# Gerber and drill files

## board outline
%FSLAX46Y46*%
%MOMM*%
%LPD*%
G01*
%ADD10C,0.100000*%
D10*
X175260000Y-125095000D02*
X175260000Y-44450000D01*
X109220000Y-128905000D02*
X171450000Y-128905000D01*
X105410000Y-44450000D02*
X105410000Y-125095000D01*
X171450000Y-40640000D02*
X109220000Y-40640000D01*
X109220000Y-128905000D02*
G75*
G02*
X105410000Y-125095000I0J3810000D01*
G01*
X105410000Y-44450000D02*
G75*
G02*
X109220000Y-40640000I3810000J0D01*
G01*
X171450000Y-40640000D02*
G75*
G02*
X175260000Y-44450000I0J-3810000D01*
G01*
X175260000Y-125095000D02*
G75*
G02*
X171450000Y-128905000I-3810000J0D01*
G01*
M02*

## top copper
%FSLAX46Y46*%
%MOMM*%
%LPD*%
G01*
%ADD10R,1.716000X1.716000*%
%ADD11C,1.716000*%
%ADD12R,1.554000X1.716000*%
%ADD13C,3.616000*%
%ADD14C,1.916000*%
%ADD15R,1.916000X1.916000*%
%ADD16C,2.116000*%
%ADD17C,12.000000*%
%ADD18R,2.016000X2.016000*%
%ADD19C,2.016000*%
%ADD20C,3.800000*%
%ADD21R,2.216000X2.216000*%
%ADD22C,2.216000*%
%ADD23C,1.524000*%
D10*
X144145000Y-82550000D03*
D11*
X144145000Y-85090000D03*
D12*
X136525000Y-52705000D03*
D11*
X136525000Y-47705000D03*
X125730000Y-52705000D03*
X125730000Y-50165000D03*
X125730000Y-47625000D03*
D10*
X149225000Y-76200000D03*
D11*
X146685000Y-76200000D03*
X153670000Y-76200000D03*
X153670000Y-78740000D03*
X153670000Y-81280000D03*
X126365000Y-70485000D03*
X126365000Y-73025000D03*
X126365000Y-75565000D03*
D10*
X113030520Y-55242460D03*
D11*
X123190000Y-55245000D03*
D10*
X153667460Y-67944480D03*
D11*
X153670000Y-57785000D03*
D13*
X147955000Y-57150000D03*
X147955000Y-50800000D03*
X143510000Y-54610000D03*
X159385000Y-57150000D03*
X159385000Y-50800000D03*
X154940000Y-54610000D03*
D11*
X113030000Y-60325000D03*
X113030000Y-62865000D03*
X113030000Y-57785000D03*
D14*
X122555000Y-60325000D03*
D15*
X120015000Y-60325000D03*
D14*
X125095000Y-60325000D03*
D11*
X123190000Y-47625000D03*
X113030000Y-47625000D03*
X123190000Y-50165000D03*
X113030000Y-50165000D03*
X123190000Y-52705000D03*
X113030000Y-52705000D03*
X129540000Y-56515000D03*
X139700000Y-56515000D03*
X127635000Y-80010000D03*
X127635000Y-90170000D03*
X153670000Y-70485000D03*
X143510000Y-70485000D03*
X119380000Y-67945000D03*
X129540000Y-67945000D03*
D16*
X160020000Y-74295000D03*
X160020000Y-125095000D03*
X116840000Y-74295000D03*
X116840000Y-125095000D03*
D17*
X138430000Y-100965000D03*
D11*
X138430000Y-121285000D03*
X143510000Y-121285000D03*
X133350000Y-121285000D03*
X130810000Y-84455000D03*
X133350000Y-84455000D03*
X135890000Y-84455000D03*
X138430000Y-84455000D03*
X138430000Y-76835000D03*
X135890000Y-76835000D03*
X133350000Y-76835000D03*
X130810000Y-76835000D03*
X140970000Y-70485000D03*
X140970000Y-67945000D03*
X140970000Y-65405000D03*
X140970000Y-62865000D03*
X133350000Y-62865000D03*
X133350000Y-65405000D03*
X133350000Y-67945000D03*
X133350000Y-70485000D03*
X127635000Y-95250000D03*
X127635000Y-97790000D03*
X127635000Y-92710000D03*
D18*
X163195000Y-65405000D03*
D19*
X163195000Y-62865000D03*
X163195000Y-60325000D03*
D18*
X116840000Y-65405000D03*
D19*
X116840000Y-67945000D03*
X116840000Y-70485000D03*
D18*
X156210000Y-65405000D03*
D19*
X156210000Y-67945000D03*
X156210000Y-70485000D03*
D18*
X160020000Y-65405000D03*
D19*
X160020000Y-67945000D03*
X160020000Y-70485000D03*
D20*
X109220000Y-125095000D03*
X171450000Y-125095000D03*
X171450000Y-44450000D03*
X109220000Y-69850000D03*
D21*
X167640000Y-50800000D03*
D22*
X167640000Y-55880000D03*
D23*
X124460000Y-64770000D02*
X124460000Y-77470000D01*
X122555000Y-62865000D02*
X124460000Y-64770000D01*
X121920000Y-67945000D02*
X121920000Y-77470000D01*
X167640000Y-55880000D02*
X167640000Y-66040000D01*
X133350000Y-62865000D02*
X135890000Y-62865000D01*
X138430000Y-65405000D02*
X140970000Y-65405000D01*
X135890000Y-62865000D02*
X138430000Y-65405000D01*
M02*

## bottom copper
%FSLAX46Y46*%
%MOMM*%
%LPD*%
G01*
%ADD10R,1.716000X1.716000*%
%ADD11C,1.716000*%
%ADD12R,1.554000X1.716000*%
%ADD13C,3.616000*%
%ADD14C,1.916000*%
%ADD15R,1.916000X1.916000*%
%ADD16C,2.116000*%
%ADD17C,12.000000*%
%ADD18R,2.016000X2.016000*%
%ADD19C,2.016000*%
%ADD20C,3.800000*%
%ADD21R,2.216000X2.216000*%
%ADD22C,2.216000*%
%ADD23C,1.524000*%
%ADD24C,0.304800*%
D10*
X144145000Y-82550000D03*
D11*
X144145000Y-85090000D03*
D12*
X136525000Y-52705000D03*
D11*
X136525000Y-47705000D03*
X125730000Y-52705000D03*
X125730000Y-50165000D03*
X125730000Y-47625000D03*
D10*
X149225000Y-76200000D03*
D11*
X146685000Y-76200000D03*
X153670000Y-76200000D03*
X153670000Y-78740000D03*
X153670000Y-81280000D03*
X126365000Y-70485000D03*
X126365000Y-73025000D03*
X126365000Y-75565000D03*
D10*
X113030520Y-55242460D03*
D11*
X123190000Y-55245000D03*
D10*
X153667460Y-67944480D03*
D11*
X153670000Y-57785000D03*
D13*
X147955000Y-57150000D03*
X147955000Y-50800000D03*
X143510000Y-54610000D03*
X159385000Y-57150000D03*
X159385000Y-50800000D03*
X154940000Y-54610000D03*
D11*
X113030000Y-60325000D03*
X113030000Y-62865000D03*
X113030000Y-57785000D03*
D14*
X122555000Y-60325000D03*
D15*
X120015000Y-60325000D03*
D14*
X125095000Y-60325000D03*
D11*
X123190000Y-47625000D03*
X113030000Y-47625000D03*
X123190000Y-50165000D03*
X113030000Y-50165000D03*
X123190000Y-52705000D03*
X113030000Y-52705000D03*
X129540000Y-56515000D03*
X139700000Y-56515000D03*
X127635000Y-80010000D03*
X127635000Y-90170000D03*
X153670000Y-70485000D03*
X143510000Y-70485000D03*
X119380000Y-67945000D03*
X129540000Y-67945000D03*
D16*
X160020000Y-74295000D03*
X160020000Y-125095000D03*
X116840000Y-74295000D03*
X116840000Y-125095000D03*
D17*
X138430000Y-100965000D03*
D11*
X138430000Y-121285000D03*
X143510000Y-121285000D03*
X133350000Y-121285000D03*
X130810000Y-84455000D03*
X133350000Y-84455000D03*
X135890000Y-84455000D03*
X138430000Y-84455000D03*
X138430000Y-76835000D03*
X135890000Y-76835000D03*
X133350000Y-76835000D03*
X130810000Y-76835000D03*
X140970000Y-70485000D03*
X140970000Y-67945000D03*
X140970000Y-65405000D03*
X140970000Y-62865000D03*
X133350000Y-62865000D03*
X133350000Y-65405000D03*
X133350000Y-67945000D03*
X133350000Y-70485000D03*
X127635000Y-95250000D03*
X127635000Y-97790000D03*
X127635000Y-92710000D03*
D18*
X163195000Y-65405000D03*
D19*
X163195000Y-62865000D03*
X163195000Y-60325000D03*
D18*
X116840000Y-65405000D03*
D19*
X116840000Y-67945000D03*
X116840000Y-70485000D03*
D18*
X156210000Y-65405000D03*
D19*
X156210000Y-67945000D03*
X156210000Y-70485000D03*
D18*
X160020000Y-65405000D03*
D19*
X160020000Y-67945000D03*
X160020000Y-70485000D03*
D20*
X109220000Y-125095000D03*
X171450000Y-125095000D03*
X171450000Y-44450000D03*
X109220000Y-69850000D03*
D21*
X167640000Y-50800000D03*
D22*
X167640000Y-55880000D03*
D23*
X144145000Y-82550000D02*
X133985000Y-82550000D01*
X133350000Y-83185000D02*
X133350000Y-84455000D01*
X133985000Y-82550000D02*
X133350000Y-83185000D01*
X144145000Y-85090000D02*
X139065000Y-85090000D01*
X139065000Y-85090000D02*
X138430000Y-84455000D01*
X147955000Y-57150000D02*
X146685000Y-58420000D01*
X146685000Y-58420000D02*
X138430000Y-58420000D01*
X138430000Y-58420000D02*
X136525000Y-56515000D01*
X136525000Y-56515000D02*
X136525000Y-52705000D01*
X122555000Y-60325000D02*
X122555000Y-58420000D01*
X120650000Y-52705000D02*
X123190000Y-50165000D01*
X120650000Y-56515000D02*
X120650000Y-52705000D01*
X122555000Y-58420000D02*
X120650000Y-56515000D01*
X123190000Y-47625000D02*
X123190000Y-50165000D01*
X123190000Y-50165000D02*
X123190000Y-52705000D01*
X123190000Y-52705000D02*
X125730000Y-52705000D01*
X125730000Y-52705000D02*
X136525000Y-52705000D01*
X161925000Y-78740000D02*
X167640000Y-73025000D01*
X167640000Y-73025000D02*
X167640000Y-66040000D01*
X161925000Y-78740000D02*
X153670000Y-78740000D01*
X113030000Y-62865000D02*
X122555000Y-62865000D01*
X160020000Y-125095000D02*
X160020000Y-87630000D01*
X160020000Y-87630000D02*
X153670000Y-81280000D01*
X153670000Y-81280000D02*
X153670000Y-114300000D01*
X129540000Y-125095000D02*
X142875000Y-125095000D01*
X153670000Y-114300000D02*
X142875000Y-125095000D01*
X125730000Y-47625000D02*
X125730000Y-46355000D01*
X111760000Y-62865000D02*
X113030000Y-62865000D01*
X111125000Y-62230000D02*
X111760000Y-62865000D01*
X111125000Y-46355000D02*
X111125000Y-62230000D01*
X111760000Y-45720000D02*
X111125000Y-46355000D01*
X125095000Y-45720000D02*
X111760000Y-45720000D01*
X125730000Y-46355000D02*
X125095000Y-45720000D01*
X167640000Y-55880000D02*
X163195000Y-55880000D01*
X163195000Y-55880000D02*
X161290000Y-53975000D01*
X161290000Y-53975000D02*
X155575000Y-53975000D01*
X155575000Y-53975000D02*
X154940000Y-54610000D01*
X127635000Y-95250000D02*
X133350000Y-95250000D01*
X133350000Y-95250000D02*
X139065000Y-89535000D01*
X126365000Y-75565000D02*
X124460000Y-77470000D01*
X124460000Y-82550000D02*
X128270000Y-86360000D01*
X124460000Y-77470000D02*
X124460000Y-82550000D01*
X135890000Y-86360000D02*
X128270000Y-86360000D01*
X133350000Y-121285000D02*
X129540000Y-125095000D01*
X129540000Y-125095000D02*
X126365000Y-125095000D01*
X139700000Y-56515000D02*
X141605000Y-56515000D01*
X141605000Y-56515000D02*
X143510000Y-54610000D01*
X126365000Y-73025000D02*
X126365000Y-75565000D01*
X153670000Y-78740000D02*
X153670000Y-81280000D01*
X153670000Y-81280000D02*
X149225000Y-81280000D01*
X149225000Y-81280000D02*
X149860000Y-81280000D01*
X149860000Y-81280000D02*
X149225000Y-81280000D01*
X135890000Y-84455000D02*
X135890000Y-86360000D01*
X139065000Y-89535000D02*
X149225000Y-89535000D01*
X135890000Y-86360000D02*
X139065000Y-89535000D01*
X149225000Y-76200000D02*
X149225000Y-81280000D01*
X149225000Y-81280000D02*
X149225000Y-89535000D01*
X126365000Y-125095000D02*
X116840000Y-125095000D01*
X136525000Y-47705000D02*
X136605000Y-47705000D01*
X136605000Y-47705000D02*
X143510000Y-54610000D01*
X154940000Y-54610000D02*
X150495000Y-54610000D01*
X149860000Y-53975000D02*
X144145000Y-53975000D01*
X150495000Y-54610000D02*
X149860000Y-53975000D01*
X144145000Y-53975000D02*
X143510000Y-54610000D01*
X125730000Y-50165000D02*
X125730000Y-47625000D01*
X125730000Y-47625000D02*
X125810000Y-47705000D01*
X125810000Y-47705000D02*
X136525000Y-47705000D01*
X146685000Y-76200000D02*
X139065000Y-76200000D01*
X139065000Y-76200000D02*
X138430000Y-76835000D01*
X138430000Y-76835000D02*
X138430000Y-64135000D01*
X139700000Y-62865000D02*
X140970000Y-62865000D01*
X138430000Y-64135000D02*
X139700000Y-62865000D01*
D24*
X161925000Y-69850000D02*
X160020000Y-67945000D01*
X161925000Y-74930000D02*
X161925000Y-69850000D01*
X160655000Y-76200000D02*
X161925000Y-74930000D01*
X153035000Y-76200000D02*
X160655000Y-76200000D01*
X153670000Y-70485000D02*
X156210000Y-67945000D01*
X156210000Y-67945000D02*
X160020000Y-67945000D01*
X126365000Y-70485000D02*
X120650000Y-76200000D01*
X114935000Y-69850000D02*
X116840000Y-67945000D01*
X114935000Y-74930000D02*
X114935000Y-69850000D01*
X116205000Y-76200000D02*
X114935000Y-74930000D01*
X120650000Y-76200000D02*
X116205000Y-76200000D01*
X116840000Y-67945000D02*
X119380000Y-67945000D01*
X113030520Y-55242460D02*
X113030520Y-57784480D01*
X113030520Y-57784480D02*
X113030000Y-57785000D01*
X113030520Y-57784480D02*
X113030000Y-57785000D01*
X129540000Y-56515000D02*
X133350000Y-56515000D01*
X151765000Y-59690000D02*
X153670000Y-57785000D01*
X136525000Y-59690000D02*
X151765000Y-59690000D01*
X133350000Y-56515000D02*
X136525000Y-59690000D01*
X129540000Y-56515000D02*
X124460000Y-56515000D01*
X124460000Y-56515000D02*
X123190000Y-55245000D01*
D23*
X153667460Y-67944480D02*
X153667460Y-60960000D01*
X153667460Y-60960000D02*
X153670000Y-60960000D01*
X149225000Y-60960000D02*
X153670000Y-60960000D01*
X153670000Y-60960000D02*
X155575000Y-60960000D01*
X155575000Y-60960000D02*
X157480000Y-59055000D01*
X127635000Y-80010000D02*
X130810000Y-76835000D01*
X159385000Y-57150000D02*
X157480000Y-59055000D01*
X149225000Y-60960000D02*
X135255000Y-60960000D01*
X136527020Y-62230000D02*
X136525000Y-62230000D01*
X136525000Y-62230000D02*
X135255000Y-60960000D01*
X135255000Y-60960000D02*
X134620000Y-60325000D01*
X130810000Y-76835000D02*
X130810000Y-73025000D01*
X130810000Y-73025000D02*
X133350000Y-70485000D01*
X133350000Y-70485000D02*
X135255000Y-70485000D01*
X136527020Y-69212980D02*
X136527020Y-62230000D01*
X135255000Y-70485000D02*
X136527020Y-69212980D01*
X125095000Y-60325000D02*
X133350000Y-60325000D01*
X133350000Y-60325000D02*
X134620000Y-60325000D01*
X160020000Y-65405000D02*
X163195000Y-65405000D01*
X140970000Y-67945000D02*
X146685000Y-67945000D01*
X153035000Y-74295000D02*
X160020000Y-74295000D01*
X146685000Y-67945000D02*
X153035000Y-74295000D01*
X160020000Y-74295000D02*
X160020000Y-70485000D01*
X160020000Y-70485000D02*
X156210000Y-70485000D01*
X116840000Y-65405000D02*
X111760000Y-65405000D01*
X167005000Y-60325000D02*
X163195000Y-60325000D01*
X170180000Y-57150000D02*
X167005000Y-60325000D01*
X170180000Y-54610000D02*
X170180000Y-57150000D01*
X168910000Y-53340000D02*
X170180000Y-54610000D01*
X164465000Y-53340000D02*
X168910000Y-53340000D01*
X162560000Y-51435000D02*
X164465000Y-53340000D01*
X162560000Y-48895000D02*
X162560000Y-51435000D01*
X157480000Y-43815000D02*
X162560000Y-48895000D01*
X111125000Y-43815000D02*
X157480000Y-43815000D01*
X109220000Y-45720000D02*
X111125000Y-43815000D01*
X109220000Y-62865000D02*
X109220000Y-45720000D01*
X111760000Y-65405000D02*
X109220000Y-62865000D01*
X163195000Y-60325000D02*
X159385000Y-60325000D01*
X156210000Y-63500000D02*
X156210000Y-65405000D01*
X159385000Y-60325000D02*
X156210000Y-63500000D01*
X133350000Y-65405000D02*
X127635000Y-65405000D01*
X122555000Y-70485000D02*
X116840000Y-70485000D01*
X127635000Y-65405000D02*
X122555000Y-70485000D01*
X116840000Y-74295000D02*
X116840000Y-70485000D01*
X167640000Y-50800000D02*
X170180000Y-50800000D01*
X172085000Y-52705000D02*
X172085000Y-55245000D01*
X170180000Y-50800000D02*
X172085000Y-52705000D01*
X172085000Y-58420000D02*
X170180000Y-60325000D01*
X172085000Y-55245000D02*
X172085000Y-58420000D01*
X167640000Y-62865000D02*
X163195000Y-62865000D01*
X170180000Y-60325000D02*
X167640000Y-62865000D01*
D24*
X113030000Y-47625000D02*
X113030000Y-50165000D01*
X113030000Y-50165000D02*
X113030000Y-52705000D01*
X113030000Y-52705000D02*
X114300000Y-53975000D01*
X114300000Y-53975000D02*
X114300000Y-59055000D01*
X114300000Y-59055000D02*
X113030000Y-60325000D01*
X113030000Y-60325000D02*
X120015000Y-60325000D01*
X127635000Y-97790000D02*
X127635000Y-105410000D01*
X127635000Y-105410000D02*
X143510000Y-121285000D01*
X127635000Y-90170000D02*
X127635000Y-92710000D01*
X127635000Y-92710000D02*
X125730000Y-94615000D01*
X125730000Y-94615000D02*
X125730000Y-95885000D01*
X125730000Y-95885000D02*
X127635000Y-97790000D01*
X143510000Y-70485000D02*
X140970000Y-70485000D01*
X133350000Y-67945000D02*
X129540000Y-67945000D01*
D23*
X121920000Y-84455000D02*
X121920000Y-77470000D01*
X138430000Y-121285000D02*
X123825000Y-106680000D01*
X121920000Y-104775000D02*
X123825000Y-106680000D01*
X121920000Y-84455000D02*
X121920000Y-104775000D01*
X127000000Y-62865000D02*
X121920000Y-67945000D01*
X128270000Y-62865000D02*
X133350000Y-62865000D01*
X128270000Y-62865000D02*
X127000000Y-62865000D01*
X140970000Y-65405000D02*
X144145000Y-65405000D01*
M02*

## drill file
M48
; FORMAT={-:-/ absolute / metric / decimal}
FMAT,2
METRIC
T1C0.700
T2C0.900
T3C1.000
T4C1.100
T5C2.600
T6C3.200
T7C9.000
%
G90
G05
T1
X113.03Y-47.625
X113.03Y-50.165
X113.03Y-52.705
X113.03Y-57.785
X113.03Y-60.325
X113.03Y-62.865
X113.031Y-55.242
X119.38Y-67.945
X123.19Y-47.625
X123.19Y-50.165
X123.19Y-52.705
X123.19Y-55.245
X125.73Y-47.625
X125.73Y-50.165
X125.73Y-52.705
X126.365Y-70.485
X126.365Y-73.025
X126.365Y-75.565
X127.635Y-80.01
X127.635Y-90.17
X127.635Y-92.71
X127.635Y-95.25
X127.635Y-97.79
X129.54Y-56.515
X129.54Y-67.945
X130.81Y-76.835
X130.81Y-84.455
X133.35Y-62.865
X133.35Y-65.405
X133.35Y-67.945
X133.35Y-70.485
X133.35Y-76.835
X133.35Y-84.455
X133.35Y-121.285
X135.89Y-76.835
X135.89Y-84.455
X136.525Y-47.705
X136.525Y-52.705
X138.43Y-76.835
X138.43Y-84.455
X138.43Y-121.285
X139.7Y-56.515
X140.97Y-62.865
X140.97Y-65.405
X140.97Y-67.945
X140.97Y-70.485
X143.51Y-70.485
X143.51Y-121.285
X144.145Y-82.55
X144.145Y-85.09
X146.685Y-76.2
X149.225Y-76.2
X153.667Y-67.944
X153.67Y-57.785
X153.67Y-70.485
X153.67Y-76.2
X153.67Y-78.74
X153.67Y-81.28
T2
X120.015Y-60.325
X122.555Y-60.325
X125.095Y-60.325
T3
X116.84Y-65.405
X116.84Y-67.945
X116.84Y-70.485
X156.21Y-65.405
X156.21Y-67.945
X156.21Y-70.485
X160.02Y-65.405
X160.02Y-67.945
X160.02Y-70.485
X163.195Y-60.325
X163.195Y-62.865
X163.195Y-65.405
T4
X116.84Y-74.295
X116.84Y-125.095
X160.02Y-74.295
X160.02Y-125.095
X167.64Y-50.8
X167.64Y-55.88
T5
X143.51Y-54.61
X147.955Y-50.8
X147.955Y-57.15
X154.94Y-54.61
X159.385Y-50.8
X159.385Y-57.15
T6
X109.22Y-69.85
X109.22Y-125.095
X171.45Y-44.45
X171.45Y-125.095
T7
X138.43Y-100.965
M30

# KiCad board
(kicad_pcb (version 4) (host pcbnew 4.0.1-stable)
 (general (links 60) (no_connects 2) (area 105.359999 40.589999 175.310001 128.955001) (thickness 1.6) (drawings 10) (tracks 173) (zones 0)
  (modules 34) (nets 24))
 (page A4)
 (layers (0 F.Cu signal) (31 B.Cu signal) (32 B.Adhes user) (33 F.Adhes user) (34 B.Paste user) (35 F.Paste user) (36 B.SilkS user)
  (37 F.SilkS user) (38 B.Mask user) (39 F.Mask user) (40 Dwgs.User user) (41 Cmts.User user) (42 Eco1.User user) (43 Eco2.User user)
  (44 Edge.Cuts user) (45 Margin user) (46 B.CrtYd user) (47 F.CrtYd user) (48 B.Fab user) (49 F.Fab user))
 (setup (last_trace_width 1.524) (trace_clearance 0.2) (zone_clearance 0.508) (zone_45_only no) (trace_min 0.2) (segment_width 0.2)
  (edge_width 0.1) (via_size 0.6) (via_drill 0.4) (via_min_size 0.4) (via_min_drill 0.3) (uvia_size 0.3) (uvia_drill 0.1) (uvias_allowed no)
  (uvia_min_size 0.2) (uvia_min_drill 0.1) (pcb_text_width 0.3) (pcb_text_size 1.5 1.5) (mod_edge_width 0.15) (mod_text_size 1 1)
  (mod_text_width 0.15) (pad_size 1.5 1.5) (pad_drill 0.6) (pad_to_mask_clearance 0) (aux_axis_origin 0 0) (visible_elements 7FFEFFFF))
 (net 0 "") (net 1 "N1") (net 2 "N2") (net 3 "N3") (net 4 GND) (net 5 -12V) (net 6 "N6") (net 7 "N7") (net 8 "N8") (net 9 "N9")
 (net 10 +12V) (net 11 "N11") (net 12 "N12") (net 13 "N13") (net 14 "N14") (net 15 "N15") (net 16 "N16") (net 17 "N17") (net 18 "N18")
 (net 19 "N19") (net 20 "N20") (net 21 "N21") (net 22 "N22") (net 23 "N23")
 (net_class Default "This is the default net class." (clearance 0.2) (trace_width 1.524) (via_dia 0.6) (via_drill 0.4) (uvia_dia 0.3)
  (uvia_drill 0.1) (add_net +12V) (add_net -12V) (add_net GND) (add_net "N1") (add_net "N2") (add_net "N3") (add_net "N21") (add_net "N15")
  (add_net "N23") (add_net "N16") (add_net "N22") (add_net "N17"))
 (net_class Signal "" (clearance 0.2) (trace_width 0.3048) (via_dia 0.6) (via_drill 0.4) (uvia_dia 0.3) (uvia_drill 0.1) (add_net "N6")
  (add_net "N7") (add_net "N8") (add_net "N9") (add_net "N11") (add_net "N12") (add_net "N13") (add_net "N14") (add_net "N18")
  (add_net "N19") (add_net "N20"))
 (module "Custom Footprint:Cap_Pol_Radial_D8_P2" (layer F.Cu) (at 144.145 82.55 270)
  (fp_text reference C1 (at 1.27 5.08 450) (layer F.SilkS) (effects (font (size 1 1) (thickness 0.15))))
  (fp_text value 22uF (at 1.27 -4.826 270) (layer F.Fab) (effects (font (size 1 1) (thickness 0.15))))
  (pad 1 thru_hole rect (at 0 0 270) (size 1.716 1.716) (drill 0.7) (layers *.Cu *.Mask F.SilkS) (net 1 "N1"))
  (pad 2 thru_hole circle (at 2.54 0 270) (size 1.716 1.716) (drill 0.7) (layers *.Cu *.Mask F.SilkS) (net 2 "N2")))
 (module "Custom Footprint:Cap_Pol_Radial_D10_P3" (layer F.Cu) (at 136.525 52.705 90)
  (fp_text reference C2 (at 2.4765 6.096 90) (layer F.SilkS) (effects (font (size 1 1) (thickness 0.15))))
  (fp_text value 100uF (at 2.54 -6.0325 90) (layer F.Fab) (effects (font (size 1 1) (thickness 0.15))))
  (pad 1 thru_hole rect (at 0 0 90) (size 1.716 1.554) (drill 0.7) (layers *.Cu *.Mask F.SilkS) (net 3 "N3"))
  (pad 2 thru_hole circle (at 5 0 90) (size 1.716 1.716) (drill 0.7) (layers *.Cu *.Mask F.SilkS) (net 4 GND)))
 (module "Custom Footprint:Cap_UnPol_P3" (layer F.Cu) (at 125.73 52.705 180)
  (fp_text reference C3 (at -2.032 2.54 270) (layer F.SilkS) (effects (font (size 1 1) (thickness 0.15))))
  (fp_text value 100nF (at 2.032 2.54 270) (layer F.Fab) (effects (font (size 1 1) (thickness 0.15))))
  (pad 1 thru_hole circle (at 0 0 180) (size 1.716 1.716) (drill 0.7) (layers *.Cu *.Mask F.SilkS) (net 3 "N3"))
  (pad 2 thru_hole circle (at 0 2.54 180) (size 1.716 1.716) (drill 0.7) (layers *.Cu *.Mask F.SilkS) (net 4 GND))
  (pad 2 thru_hole circle (at 0 5.08 180) (size 1.716 1.716) (drill 0.7) (layers *.Cu *.Mask F.SilkS) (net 4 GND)))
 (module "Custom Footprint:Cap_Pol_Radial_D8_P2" (layer F.Cu) (at 149.225 76.2 180)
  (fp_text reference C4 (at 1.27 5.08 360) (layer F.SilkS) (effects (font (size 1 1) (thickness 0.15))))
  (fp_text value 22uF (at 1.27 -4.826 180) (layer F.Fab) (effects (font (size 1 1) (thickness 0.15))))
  (pad 1 thru_hole rect (at 0 0 180) (size 1.716 1.716) (drill 0.7) (layers *.Cu *.Mask F.SilkS) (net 4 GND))
  (pad 2 thru_hole circle (at 2.54 0 180) (size 1.716 1.716) (drill 0.7) (layers *.Cu *.Mask F.SilkS) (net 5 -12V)))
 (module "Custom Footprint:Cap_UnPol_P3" (layer F.Cu) (at 153.67 76.2)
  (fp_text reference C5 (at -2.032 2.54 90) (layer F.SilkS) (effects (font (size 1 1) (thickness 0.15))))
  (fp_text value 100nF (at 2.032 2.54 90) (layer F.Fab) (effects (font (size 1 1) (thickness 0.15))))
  (pad 1 thru_hole circle (at 0 0) (size 1.716 1.716) (drill 0.7) (layers *.Cu *.Mask F.SilkS) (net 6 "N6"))
  (pad 2 thru_hole circle (at 0 2.54) (size 1.716 1.716) (drill 0.7) (layers *.Cu *.Mask F.SilkS) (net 4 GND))
  (pad 2 thru_hole circle (at 0 5.08) (size 1.716 1.716) (drill 0.7) (layers *.Cu *.Mask F.SilkS) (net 4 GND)))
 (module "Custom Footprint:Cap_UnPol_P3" (layer F.Cu) (at 126.365 70.485)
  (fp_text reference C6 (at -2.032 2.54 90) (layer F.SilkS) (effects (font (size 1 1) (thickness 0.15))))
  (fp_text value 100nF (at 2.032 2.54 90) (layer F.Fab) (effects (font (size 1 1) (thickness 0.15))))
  (pad 1 thru_hole circle (at 0 0) (size 1.716 1.716) (drill 0.7) (layers *.Cu *.Mask F.SilkS) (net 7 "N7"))
  (pad 2 thru_hole circle (at 0 2.54) (size 1.716 1.716) (drill 0.7) (layers *.Cu *.Mask F.SilkS) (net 4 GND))
  (pad 2 thru_hole circle (at 0 5.08) (size 1.716 1.716) (drill 0.7) (layers *.Cu *.Mask F.SilkS) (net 4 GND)))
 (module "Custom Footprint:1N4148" (layer F.Cu) (at 113.03 55.245)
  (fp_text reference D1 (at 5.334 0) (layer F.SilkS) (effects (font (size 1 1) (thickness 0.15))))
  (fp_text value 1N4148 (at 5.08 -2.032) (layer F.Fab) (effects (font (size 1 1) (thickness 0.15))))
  (pad 1 thru_hole rect (at 0.00052 -0.00254 180) (size 1.716 1.716) (drill 0.7) (layers *.Cu *.Mask F.SilkS) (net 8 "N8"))
  (pad 2 thru_hole circle (at 10.16 0) (size 1.716 1.716) (drill 0.7) (layers *.Cu *.Mask F.SilkS) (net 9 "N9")))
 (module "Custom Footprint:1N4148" (layer F.Cu) (at 153.67 67.945 90)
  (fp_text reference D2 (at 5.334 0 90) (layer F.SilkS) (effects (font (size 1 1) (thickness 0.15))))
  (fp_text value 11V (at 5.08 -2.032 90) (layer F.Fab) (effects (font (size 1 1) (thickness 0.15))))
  (pad 1 thru_hole rect (at 0.00052 -0.00254 270) (size 1.716 1.716) (drill 0.7) (layers *.Cu *.Mask F.SilkS) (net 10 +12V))
  (pad 2 thru_hole circle (at 10.16 0 90) (size 1.716 1.716) (drill 0.7) (layers *.Cu *.Mask F.SilkS) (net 9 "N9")))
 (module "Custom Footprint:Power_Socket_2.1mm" (layer F.Cu) (at 147.955 50.8)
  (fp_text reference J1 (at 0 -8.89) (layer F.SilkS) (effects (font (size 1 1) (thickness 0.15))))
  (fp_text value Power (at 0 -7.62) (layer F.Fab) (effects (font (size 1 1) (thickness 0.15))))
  (pad 1 thru_hole circle (at 0 6.35) (size 3.616 3.616) (drill 2.6) (layers *.Cu *.Mask F.SilkS) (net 3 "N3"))
  (pad 3 thru_hole circle (at 0 0) (size 3.616 3.616) (drill 2.6) (layers *.Cu *.Mask F.SilkS))
  (pad 2 thru_hole circle (at -4.445 3.81) (size 3.616 3.616) (drill 2.6) (layers *.Cu *.Mask F.SilkS) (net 4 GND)))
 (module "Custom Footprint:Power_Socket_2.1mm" (layer F.Cu) (at 159.385 50.8)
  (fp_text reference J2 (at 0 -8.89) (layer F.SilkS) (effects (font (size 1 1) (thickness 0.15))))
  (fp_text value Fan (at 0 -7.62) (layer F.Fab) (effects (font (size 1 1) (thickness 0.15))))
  (pad 1 thru_hole circle (at 0 6.35) (size 3.616 3.616) (drill 2.6) (layers *.Cu *.Mask F.SilkS) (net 10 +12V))
  (pad 3 thru_hole circle (at 0 0) (size 3.616 3.616) (drill 2.6) (layers *.Cu *.Mask F.SilkS))
  (pad 2 thru_hole circle (at -4.445 3.81) (size 3.616 3.616) (drill 2.6) (layers *.Cu *.Mask F.SilkS) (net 4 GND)))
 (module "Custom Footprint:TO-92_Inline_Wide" (layer F.Cu) (at 113.03 57.785 270)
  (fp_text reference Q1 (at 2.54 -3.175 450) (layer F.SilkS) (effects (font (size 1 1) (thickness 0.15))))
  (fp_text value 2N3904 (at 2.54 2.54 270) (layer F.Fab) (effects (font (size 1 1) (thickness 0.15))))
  (pad 2 thru_hole circle (at 2.54 0) (size 1.716 1.716) (drill 0.7) (layers *.Cu *.Mask F.SilkS) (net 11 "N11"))
  (pad 3 thru_hole circle (at 5.08 0) (size 1.716 1.716) (drill 0.7) (layers *.Cu *.Mask F.SilkS) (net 4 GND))
  (pad 1 thru_hole circle (at 0 0) (size 1.716 1.716) (drill 0.7) (layers *.Cu *.Mask F.SilkS) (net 8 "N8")))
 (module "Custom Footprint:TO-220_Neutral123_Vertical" (layer F.Cu) (at 122.555 60.325)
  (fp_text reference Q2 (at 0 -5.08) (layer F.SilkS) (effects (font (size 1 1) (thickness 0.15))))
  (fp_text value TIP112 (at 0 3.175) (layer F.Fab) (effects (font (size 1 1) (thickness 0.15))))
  (pad 2 thru_hole circle (at 0 0 90) (size 1.916 1.916) (drill 0.9) (layers *.Cu *.Mask F.SilkS) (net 3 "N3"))
  (pad 1 thru_hole rect (at -2.54 0 90) (size 1.916 1.916) (drill 0.9) (layers *.Cu *.Mask F.SilkS) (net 11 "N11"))
  (pad 3 thru_hole circle (at 2.54 0 90) (size 1.916 1.916) (drill 0.9) (layers *.Cu *.Mask F.SilkS) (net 10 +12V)))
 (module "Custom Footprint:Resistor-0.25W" (layer F.Cu) (at 123.19 47.625 180)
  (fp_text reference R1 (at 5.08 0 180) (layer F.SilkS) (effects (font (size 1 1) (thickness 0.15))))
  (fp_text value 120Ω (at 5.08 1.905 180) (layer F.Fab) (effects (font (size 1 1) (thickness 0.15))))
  (pad 1 thru_hole circle (at 0 0 180) (size 1.716 1.716) (drill 0.7) (layers *.Cu *.Mask F.SilkS) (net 3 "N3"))
  (pad 2 thru_hole circle (at 10.16 0 180) (size 1.716 1.716) (drill 0.7) (layers *.Cu *.Mask F.SilkS) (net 11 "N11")))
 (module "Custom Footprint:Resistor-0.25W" (layer F.Cu) (at 123.19 50.165 180)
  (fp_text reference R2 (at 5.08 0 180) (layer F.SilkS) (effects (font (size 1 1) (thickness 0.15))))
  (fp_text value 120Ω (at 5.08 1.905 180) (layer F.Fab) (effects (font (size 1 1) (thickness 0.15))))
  (pad 1 thru_hole circle (at 0 0 180) (size 1.716 1.716) (drill 0.7) (layers *.Cu *.Mask F.SilkS) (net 3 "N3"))
  (pad 2 thru_hole circle (at 10.16 0 180) (size 1.716 1.716) (drill 0.7) (layers *.Cu *.Mask F.SilkS) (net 11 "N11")))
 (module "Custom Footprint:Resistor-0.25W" (layer F.Cu) (at 123.19 52.705 180)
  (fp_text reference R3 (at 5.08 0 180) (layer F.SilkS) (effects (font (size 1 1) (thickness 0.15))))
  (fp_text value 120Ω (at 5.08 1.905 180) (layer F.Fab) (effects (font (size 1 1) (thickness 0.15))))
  (pad 1 thru_hole circle (at 0 0 180) (size 1.716 1.716) (drill 0.7) (layers *.Cu *.Mask F.SilkS) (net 3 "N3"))
  (pad 2 thru_hole circle (at 10.16 0 180) (size 1.716 1.716) (drill 0.7) (layers *.Cu *.Mask F.SilkS) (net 11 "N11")))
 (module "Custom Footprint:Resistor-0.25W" (layer F.Cu) (at 129.54 56.515)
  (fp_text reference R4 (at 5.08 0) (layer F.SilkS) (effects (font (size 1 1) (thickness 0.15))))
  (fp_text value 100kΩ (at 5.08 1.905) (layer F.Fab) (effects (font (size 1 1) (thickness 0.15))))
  (pad 1 thru_hole circle (at 0 0) (size 1.716 1.716) (drill 0.7) (layers *.Cu *.Mask F.SilkS) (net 9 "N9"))
  (pad 2 thru_hole circle (at 10.16 0) (size 1.716 1.716) (drill 0.7) (layers *.Cu *.Mask F.SilkS) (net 4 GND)))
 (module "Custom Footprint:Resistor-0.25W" (layer F.Cu) (at 127.635 80.01 270)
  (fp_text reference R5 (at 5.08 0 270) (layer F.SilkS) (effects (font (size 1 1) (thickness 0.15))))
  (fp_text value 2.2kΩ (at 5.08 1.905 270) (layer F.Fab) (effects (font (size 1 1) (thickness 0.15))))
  (pad 1 thru_hole circle (at 0 0 270) (size 1.716 1.716) (drill 0.7) (layers *.Cu *.Mask F.SilkS) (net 10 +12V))
  (pad 2 thru_hole circle (at 10.16 0 270) (size 1.716 1.716) (drill 0.7) (layers *.Cu *.Mask F.SilkS) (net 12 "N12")))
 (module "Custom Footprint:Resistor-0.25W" (layer F.Cu) (at 153.67 70.485 180)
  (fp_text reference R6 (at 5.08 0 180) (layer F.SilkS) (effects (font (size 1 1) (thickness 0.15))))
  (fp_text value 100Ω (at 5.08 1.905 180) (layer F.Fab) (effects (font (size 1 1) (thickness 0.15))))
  (pad 1 thru_hole circle (at 0 0 180) (size 1.716 1.716) (drill 0.7) (layers *.Cu *.Mask F.SilkS) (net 6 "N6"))
  (pad 2 thru_hole circle (at 10.16 0 180) (size 1.716 1.716) (drill 0.7) (layers *.Cu *.Mask F.SilkS) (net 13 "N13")))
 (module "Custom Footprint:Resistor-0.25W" (layer F.Cu) (at 119.38 67.945)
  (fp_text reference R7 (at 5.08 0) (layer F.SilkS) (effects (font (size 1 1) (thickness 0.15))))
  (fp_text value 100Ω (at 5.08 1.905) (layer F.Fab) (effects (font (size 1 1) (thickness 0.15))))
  (pad 1 thru_hole circle (at 0 0) (size 1.716 1.716) (drill 0.7) (layers *.Cu *.Mask F.SilkS) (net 7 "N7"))
  (pad 2 thru_hole circle (at 10.16 0) (size 1.716 1.716) (drill 0.7) (layers *.Cu *.Mask F.SilkS) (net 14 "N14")))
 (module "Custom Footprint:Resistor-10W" (layer F.Cu) (at 160.02 99.695 270)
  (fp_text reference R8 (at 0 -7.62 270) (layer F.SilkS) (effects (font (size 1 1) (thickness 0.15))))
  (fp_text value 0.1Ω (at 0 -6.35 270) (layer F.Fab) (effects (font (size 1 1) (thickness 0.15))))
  (pad 1 thru_hole circle (at -25.4 0 270) (size 2.116 2.116) (drill 1.1) (layers *.Cu *.Mask F.SilkS) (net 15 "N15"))
  (pad 2 thru_hole circle (at 25.4 0 270) (size 2.116 2.116) (drill 1.1) (layers *.Cu *.Mask F.SilkS) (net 4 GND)))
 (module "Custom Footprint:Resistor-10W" (layer F.Cu) (at 116.84 99.695 270)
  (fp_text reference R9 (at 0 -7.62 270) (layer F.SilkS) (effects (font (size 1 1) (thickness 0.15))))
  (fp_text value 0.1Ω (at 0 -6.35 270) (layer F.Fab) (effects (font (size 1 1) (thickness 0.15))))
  (pad 1 thru_hole circle (at -25.4 0 270) (size 2.116 2.116) (drill 1.1) (layers *.Cu *.Mask F.SilkS) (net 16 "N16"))
  (pad 2 thru_hole circle (at 25.4 0 270) (size 2.116 2.116) (drill 1.1) (layers *.Cu *.Mask F.SilkS) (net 4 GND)))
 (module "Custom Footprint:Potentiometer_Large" (layer F.Cu) (at 138.43 100.965)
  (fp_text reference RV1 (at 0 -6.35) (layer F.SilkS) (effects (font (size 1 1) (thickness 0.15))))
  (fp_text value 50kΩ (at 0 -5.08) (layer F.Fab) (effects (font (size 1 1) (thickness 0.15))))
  (pad "" thru_hole circle (at 0 0) (size 12 12) (drill 9) (layers *.Cu *.Mask F.SilkS))
  (pad 2 thru_hole circle (at 0 20.32) (size 1.716 1.716) (drill 0.7) (layers *.Cu *.Mask F.SilkS) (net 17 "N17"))
  (pad 3 thru_hole circle (at 5.08 20.32) (size 1.716 1.716) (drill 0.7) (layers *.Cu *.Mask F.SilkS) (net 12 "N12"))
  (pad 1 thru_hole circle (at -5.08 20.32) (size 1.716 1.716) (drill 0.7) (layers *.Cu *.Mask F.SilkS) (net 4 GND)))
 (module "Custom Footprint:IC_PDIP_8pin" (layer F.Cu) (at 134.62 80.645)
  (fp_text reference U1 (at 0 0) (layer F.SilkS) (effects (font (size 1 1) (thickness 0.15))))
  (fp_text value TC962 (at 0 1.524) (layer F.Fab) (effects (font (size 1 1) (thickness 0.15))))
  (pad 1 thru_hole circle (at -3.81 3.81) (size 1.716 1.716) (drill 0.7) (layers *.Cu *.Mask F.SilkS) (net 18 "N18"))
  (pad 2 thru_hole circle (at -1.27 3.81) (size 1.716 1.716) (drill 0.7) (layers *.Cu *.Mask F.SilkS) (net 1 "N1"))
  (pad 3 thru_hole circle (at 1.27 3.81) (size 1.716 1.716) (drill 0.7) (layers *.Cu *.Mask F.SilkS) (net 4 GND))
  (pad 4 thru_hole circle (at 3.81 3.81) (size 1.716 1.716) (drill 0.7) (layers *.Cu *.Mask F.SilkS) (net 2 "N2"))
  (pad 5 thru_hole circle (at 3.81 -3.81) (size 1.716 1.716) (drill 0.7) (layers *.Cu *.Mask F.SilkS) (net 5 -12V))
  (pad 6 thru_hole circle (at 1.27 -3.81) (size 1.716 1.716) (drill 0.7) (layers *.Cu *.Mask F.SilkS) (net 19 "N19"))
  (pad 7 thru_hole circle (at -1.27 -3.81) (size 1.716 1.716) (drill 0.7) (layers *.Cu *.Mask F.SilkS) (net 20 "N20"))
  (pad 8 thru_hole circle (at -3.81 -3.81) (size 1.716 1.716) (drill 0.7) (layers *.Cu *.Mask F.SilkS) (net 10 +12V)))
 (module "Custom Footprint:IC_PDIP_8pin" (layer F.Cu) (at 137.16 66.675 90)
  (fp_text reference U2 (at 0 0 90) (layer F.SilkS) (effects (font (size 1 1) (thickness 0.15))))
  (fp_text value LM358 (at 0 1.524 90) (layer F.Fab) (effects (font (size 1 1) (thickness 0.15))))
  (pad 1 thru_hole circle (at -3.81 3.81 90) (size 1.716 1.716) (drill 0.7) (layers *.Cu *.Mask F.SilkS) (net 13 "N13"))
  (pad 2 thru_hole circle (at -1.27 3.81 90) (size 1.716 1.716) (drill 0.7) (layers *.Cu *.Mask F.SilkS) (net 15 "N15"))
  (pad 3 thru_hole circle (at 1.27 3.81 90) (size 1.716 1.716) (drill 0.7) (layers *.Cu *.Mask F.SilkS) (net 17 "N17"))
  (pad 4 thru_hole circle (at 3.81 3.81 90) (size 1.716 1.716) (drill 0.7) (layers *.Cu *.Mask F.SilkS) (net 5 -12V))
  (pad 5 thru_hole circle (at 3.81 -3.81 90) (size 1.716 1.716) (drill 0.7) (layers *.Cu *.Mask F.SilkS) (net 17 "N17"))
  (pad 6 thru_hole circle (at 1.27 -3.81 90) (size 1.716 1.716) (drill 0.7) (layers *.Cu *.Mask F.SilkS) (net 16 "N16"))
  (pad 7 thru_hole circle (at -1.27 -3.81 90) (size 1.716 1.716) (drill 0.7) (layers *.Cu *.Mask F.SilkS) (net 14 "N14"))
  (pad 8 thru_hole circle (at -3.81 -3.81 90) (size 1.716 1.716) (drill 0.7) (layers *.Cu *.Mask F.SilkS) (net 10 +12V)))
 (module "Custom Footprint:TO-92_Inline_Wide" (layer F.Cu) (at 127.635 92.71 270)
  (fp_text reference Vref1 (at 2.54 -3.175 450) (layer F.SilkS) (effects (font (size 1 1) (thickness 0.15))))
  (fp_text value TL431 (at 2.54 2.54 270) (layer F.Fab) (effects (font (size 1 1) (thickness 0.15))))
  (pad 2 thru_hole circle (at 2.54 0) (size 1.716 1.716) (drill 0.7) (layers *.Cu *.Mask F.SilkS) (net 4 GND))
  (pad 3 thru_hole circle (at 5.08 0) (size 1.716 1.716) (drill 0.7) (layers *.Cu *.Mask F.SilkS) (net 12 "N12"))
  (pad 1 thru_hole circle (at 0 0) (size 1.716 1.716) (drill 0.7) (layers *.Cu *.Mask F.SilkS) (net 12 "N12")))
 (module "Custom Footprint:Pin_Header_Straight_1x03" (layer F.Cu) (at 163.195 65.405 180)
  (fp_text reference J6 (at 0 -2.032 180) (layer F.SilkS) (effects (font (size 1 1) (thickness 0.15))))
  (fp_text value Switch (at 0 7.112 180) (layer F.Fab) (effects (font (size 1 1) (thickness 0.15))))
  (pad 1 thru_hole rect (at 0 0 180) (size 2.016 2.016) (drill 1) (layers *.Cu *.Mask F.SilkS) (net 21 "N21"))
  (pad 2 thru_hole circle (at 0 2.54 180) (size 2.016 2.016) (drill 1) (layers *.Cu *.Mask F.SilkS) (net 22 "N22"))
  (pad 3 thru_hole circle (at 0 5.08 180) (size 2.016 2.016) (drill 1) (layers *.Cu *.Mask F.SilkS) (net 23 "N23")))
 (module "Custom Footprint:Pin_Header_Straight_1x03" (layer F.Cu) (at 116.84 65.405)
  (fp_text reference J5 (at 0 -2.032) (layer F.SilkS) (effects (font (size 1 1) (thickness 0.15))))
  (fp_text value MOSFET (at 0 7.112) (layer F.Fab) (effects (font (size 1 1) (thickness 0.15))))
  (pad 1 thru_hole rect (at 0 0) (size 2.016 2.016) (drill 1) (layers *.Cu *.Mask F.SilkS) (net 23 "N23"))
  (pad 2 thru_hole circle (at 0 2.54) (size 2.016 2.016) (drill 1) (layers *.Cu *.Mask F.SilkS) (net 7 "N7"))
  (pad 3 thru_hole circle (at 0 5.08) (size 2.016 2.016) (drill 1) (layers *.Cu *.Mask F.SilkS) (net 16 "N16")))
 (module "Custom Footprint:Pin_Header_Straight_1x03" (layer F.Cu) (at 156.21 65.405)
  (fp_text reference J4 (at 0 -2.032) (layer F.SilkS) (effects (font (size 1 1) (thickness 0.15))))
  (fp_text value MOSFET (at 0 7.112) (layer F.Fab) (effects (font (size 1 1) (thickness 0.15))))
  (pad 1 thru_hole rect (at 0 0) (size 2.016 2.016) (drill 1) (layers *.Cu *.Mask F.SilkS) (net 23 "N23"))
  (pad 2 thru_hole circle (at 0 2.54) (size 2.016 2.016) (drill 1) (layers *.Cu *.Mask F.SilkS) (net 6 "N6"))
  (pad 3 thru_hole circle (at 0 5.08) (size 2.016 2.016) (drill 1) (layers *.Cu *.Mask F.SilkS) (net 15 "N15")))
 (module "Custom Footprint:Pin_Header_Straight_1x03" (layer F.Cu) (at 160.02 65.405)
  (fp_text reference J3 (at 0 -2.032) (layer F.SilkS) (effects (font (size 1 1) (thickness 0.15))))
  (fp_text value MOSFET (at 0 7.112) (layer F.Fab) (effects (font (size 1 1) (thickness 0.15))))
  (pad 1 thru_hole rect (at 0 0) (size 2.016 2.016) (drill 1) (layers *.Cu *.Mask F.SilkS) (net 21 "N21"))
  (pad 2 thru_hole circle (at 0 2.54) (size 2.016 2.016) (drill 1) (layers *.Cu *.Mask F.SilkS) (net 6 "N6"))
  (pad 3 thru_hole circle (at 0 5.08) (size 2.016 2.016) (drill 1) (layers *.Cu *.Mask F.SilkS) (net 15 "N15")))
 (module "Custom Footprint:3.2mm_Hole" (layer F.Cu) (at 109.22 125.095)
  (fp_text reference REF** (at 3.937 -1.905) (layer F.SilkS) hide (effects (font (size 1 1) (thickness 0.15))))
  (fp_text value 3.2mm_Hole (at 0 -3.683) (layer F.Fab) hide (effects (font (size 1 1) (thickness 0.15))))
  (pad 1 thru_hole circle (at 0 0) (size 3.8 3.8) (drill 3.2) (layers *.Cu *.Mask F.SilkS)))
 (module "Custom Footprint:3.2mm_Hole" (layer F.Cu) (at 171.45 125.095)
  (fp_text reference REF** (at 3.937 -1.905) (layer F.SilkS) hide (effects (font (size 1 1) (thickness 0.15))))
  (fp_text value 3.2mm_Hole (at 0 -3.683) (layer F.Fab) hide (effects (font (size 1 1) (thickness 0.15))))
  (pad 1 thru_hole circle (at 0 0) (size 3.8 3.8) (drill 3.2) (layers *.Cu *.Mask F.SilkS)))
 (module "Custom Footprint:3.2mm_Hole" (layer F.Cu) (at 171.45 44.45)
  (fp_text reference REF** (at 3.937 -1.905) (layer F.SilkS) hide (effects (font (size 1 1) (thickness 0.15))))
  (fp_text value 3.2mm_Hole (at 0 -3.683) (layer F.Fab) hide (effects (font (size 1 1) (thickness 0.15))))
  (pad 1 thru_hole circle (at 0 0) (size 3.8 3.8) (drill 3.2) (layers *.Cu *.Mask F.SilkS)))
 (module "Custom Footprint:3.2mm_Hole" (layer F.Cu) (at 109.22 69.85)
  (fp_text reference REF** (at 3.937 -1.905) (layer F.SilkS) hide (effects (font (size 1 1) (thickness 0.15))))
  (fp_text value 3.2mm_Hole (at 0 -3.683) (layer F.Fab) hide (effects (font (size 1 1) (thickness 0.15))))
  (pad 1 thru_hole circle (at 0 0) (size 3.8 3.8) (drill 3.2) (layers *.Cu *.Mask F.SilkS)))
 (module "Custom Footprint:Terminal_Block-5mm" (layer F.Cu) (at 167.64 53.34 270)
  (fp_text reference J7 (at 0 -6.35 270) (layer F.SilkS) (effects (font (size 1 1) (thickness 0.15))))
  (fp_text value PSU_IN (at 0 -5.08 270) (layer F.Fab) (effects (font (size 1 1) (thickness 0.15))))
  (pad 1 thru_hole rect (at -2.54 0 270) (size 2.216 2.216) (drill 1.1) (layers *.Cu *.Mask F.SilkS) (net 22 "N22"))
  (pad 2 thru_hole circle (at 2.54 0 270) (size 2.216 2.216) (drill 1.1) (layers *.Cu *.Mask F.SilkS) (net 4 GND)))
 (gr_line (start 175.26 125.095) (end 175.26 44.45) (angle 90) (layer Edge.Cuts) (width 0.1))
 (gr_line (start 109.22 128.905) (end 171.45 128.905) (angle 90) (layer Edge.Cuts) (width 0.1))
 (gr_line (start 105.41 44.45) (end 105.41 125.095) (angle 90) (layer Edge.Cuts) (width 0.1))
 (gr_line (start 171.45 40.64) (end 109.22 40.64) (angle 90) (layer Edge.Cuts) (width 0.1))
 (gr_arc (start 109.22 125.095) (end 109.22 128.905) (angle 90) (layer Edge.Cuts) (width 0.1))
 (gr_arc (start 109.22 44.45) (end 105.41 44.45) (angle 90) (layer Edge.Cuts) (width 0.1))
 (gr_arc (start 171.45 44.45) (end 171.45 40.64) (angle 90) (layer Edge.Cuts) (width 0.1))
 (gr_arc (start 171.45 125.095) (end 175.26 125.095) (angle 90) (layer Edge.Cuts) (width 0.1))
 (segment (start 124.46 64.77) (end 124.46 77.47) (width 1.524) (layer F.Cu) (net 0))
 (segment (start 122.555 62.865) (end 124.46 64.77) (width 1.524) (layer F.Cu) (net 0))
 (segment (start 121.92 67.945) (end 121.92 77.47) (width 1.524) (layer F.Cu) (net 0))
 (segment (start 144.145 82.55) (end 133.985 82.55) (width 1.524) (layer B.Cu) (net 1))
 (segment (start 133.35 83.185) (end 133.35 84.455) (width 1.524) (layer B.Cu) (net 1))
 (segment (start 133.985 82.55) (end 133.35 83.185) (width 1.524) (layer B.Cu) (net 1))
 (segment (start 144.145 85.09) (end 139.065 85.09) (width 1.524) (layer B.Cu) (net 2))
 (segment (start 139.065 85.09) (end 138.43 84.455) (width 1.524) (layer B.Cu) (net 2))
 (segment (start 147.955 57.15) (end 146.685 58.42) (width 1.524) (layer B.Cu) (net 3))
 (segment (start 146.685 58.42) (end 138.43 58.42) (width 1.524) (layer B.Cu) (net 3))
 (segment (start 138.43 58.42) (end 136.525 56.515) (width 1.524) (layer B.Cu) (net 3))
 (segment (start 136.525 56.515) (end 136.525 52.705) (width 1.524) (layer B.Cu) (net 3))
 (segment (start 122.555 60.325) (end 122.555 58.42) (width 1.524) (layer B.Cu) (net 3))
 (segment (start 120.65 52.705) (end 123.19 50.165) (width 1.524) (layer B.Cu) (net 3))
 (segment (start 120.65 56.515) (end 120.65 52.705) (width 1.524) (layer B.Cu) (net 3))
 (segment (start 122.555 58.42) (end 120.65 56.515) (width 1.524) (layer B.Cu) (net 3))
 (segment (start 123.19 47.625) (end 123.19 50.165) (width 1.524) (layer B.Cu) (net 3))
 (segment (start 123.19 50.165) (end 123.19 52.705) (width 1.524) (layer B.Cu) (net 3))
 (segment (start 123.19 52.705) (end 125.73 52.705) (width 1.524) (layer B.Cu) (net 3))
 (segment (start 125.73 52.705) (end 136.525 52.705) (width 1.524) (layer B.Cu) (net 3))
 (segment (start 167.64 55.88) (end 167.64 66.04) (width 1.524) (layer F.Cu) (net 4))
 (segment (start 161.925 78.74) (end 167.64 73.025) (width 1.524) (layer B.Cu) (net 4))
 (segment (start 167.64 73.025) (end 167.64 66.04) (width 1.524) (layer B.Cu) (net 4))
 (segment (start 161.925 78.74) (end 153.67 78.74) (width 1.524) (layer B.Cu) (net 4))
 (segment (start 113.03 62.865) (end 122.555 62.865) (width 1.524) (layer B.Cu) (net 4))
 (segment (start 160.02 125.095) (end 160.02 87.63) (width 1.524) (layer B.Cu) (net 4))
 (segment (start 160.02 87.63) (end 153.67 81.28) (width 1.524) (layer B.Cu) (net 4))
 (segment (start 153.67 81.28) (end 153.67 114.3) (width 1.524) (layer B.Cu) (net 4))
 (segment (start 129.54 125.095) (end 142.875 125.095) (width 1.524) (layer B.Cu) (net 4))
 (segment (start 153.67 114.3) (end 142.875 125.095) (width 1.524) (layer B.Cu) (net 4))
 (segment (start 125.73 47.625) (end 125.73 46.355) (width 1.524) (layer B.Cu) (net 4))
 (segment (start 111.76 62.865) (end 113.03 62.865) (width 1.524) (layer B.Cu) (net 4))
 (segment (start 111.125 62.23) (end 111.76 62.865) (width 1.524) (layer B.Cu) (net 4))
 (segment (start 111.125 46.355) (end 111.125 62.23) (width 1.524) (layer B.Cu) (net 4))
 (segment (start 111.76 45.72) (end 111.125 46.355) (width 1.524) (layer B.Cu) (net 4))
 (segment (start 125.095 45.72) (end 111.76 45.72) (width 1.524) (layer B.Cu) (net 4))
 (segment (start 125.73 46.355) (end 125.095 45.72) (width 1.524) (layer B.Cu) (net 4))
 (segment (start 167.64 55.88) (end 163.195 55.88) (width 1.524) (layer B.Cu) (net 4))
 (segment (start 163.195 55.88) (end 161.29 53.975) (width 1.524) (layer B.Cu) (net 4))
 (segment (start 161.29 53.975) (end 155.575 53.975) (width 1.524) (layer B.Cu) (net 4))
 (segment (start 155.575 53.975) (end 154.94 54.61) (width 1.524) (layer B.Cu) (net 4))
 (segment (start 127.635 95.25) (end 133.35 95.25) (width 1.524) (layer B.Cu) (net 4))
 (segment (start 133.35 95.25) (end 139.065 89.535) (width 1.524) (layer B.Cu) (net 4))
 (segment (start 126.365 75.565) (end 124.46 77.47) (width 1.524) (layer B.Cu) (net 4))
 (segment (start 124.46 82.55) (end 128.27 86.36) (width 1.524) (layer B.Cu) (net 4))
 (segment (start 124.46 77.47) (end 124.46 82.55) (width 1.524) (layer B.Cu) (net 4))
 (segment (start 135.89 86.36) (end 128.27 86.36) (width 1.524) (layer B.Cu) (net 4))
 (segment (start 133.35 121.285) (end 129.54 125.095) (width 1.524) (layer B.Cu) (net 4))
 (segment (start 129.54 125.095) (end 126.365 125.095) (width 1.524) (layer B.Cu) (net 4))
 (segment (start 139.7 56.515) (end 141.605 56.515) (width 1.524) (layer B.Cu) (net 4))
 (segment (start 141.605 56.515) (end 143.51 54.61) (width 1.524) (layer B.Cu) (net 4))
 (segment (start 126.365 73.025) (end 126.365 75.565) (width 1.524) (layer B.Cu) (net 4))
 (segment (start 153.67 78.74) (end 153.67 81.28) (width 1.524) (layer B.Cu) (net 4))
 (segment (start 153.67 81.28) (end 149.225 81.28) (width 1.524) (layer B.Cu) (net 4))
 (segment (start 149.225 81.28) (end 149.86 81.28) (width 1.524) (layer B.Cu) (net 4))
 (segment (start 149.86 81.28) (end 149.225 81.28) (width 1.524) (layer B.Cu) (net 4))
 (segment (start 135.89 84.455) (end 135.89 86.36) (width 1.524) (layer B.Cu) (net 4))
 (segment (start 139.065 89.535) (end 149.225 89.535) (width 1.524) (layer B.Cu) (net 4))
 (segment (start 135.89 86.36) (end 139.065 89.535) (width 1.524) (layer B.Cu) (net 4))
 (segment (start 149.225 76.2) (end 149.225 81.28) (width 1.524) (layer B.Cu) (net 4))
 (segment (start 149.225 81.28) (end 149.225 89.535) (width 1.524) (layer B.Cu) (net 4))
 (segment (start 126.365 125.095) (end 116.84 125.095) (width 1.524) (layer B.Cu) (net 4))
 (segment (start 136.525 47.705) (end 136.605 47.705) (width 1.524) (layer B.Cu) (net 4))
 (segment (start 136.605 47.705) (end 143.51 54.61) (width 1.524) (layer B.Cu) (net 4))
 (segment (start 154.94 54.61) (end 150.495 54.61) (width 1.524) (layer B.Cu) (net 4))
 (segment (start 149.86 53.975) (end 144.145 53.975) (width 1.524) (layer B.Cu) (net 4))
 (segment (start 150.495 54.61) (end 149.86 53.975) (width 1.524) (layer B.Cu) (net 4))
 (segment (start 144.145 53.975) (end 143.51 54.61) (width 1.524) (layer B.Cu) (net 4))
 (segment (start 125.73 50.165) (end 125.73 47.625) (width 1.524) (layer B.Cu) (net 4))
 (segment (start 125.73 47.625) (end 125.81 47.705) (width 1.524) (layer B.Cu) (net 4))
 (segment (start 125.81 47.705) (end 136.525 47.705) (width 1.524) (layer B.Cu) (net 4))
 (segment (start 146.685 76.2) (end 139.065 76.2) (width 1.524) (layer B.Cu) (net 5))
 (segment (start 139.065 76.2) (end 138.43 76.835) (width 1.524) (layer B.Cu) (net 5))
 (segment (start 138.43 76.835) (end 138.43 64.135) (width 1.524) (layer B.Cu) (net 5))
 (segment (start 139.7 62.865) (end 140.97 62.865) (width 1.524) (layer B.Cu) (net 5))
 (segment (start 138.43 64.135) (end 139.7 62.865) (width 1.524) (layer B.Cu) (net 5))
 (segment (start 161.925 69.85) (end 160.02 67.945) (width 0.3048) (layer B.Cu) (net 6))
 (segment (start 161.925 74.93) (end 161.925 69.85) (width 0.3048) (layer B.Cu) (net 6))
 (segment (start 160.655 76.2) (end 161.925 74.93) (width 0.3048) (layer B.Cu) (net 6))
 (segment (start 153.035 76.2) (end 160.655 76.2) (width 0.3048) (layer B.Cu) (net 6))
 (segment (start 153.67 70.485) (end 156.21 67.945) (width 0.3048) (layer B.Cu) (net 6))
 (segment (start 156.21 67.945) (end 160.02 67.945) (width 0.3048) (layer B.Cu) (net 6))
 (segment (start 126.365 70.485) (end 120.65 76.2) (width 0.3048) (layer B.Cu) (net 7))
 (segment (start 114.935 69.85) (end 116.84 67.945) (width 0.3048) (layer B.Cu) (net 7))
 (segment (start 114.935 74.93) (end 114.935 69.85) (width 0.3048) (layer B.Cu) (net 7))
 (segment (start 116.205 76.2) (end 114.935 74.93) (width 0.3048) (layer B.Cu) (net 7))
 (segment (start 120.65 76.2) (end 116.205 76.2) (width 0.3048) (layer B.Cu) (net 7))
 (segment (start 116.84 67.945) (end 119.38 67.945) (width 0.3048) (layer B.Cu) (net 7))
 (segment (start 113.03052 55.24246) (end 113.03052 57.78448) (width 0.3048) (layer B.Cu) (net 8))
 (segment (start 113.03052 57.78448) (end 113.03 57.785) (width 0.3048) (layer B.Cu) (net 8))
 (segment (start 113.03052 57.78448) (end 113.03 57.785) (width 0.3048) (layer B.Cu) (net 8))
 (segment (start 129.54 56.515) (end 133.35 56.515) (width 0.3048) (layer B.Cu) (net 9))
 (segment (start 151.765 59.69) (end 153.67 57.785) (width 0.3048) (layer B.Cu) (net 9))
 (segment (start 136.525 59.69) (end 151.765 59.69) (width 0.3048) (layer B.Cu) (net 9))
 (segment (start 133.35 56.515) (end 136.525 59.69) (width 0.3048) (layer B.Cu) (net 9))
 (segment (start 129.54 56.515) (end 124.46 56.515) (width 0.3048) (layer B.Cu) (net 9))
 (segment (start 124.46 56.515) (end 123.19 55.245) (width 0.3048) (layer B.Cu) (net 9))
 (segment (start 153.66746 67.94448) (end 153.66746 60.96) (width 1.524) (layer B.Cu) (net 10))
 (segment (start 153.66746 60.96) (end 153.67 60.96) (width 1.524) (layer B.Cu) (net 10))
 (segment (start 149.225 60.96) (end 153.67 60.96) (width 1.524) (layer B.Cu) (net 10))
 (segment (start 153.67 60.96) (end 155.575 60.96) (width 1.524) (layer B.Cu) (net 10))
 (segment (start 155.575 60.96) (end 157.48 59.055) (width 1.524) (layer B.Cu) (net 10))
 (segment (start 127.635 80.01) (end 130.81 76.835) (width 1.524) (layer B.Cu) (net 10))
 (segment (start 159.385 57.15) (end 157.48 59.055) (width 1.524) (layer B.Cu) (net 10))
 (segment (start 149.225 60.96) (end 135.255 60.96) (width 1.524) (layer B.Cu) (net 10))
 (segment (start 136.52702 62.23) (end 136.525 62.23) (width 1.524) (layer B.Cu) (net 10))
 (segment (start 136.525 62.23) (end 135.255 60.96) (width 1.524) (layer B.Cu) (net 10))
 (segment (start 135.255 60.96) (end 134.62 60.325) (width 1.524) (layer B.Cu) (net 10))
 (segment (start 130.81 76.835) (end 130.81 73.025) (width 1.524) (layer B.Cu) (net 10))
 (segment (start 130.81 73.025) (end 133.35 70.485) (width 1.524) (layer B.Cu) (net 10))
 (segment (start 133.35 70.485) (end 135.255 70.485) (width 1.524) (layer B.Cu) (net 10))
 (segment (start 136.52702 69.21298) (end 136.52702 62.23) (width 1.524) (layer B.Cu) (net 10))
 (segment (start 135.255 70.485) (end 136.52702 69.21298) (width 1.524) (layer B.Cu) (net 10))
 (segment (start 125.095 60.325) (end 133.35 60.325) (width 1.524) (layer B.Cu) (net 10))
 (segment (start 133.35 60.325) (end 134.62 60.325) (width 1.524) (layer B.Cu) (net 10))
 (segment (start 160.02 65.405) (end 163.195 65.405) (width 1.524) (layer B.Cu) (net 21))
 (segment (start 140.97 67.945) (end 146.685 67.945) (width 1.524) (layer B.Cu) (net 15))
 (segment (start 153.035 74.295) (end 160.02 74.295) (width 1.524) (layer B.Cu) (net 15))
 (segment (start 146.685 67.945) (end 153.035 74.295) (width 1.524) (layer B.Cu) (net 15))
 (segment (start 160.02 74.295) (end 160.02 70.485) (width 1.524) (layer B.Cu) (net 15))
 (segment (start 160.02 70.485) (end 156.21 70.485) (width 1.524) (layer B.Cu) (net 15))
 (segment (start 116.84 65.405) (end 111.76 65.405) (width 1.524) (layer B.Cu) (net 23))
 (segment (start 167.005 60.325) (end 163.195 60.325) (width 1.524) (layer B.Cu) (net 23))
 (segment (start 170.18 57.15) (end 167.005 60.325) (width 1.524) (layer B.Cu) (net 23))
 (segment (start 170.18 54.61) (end 170.18 57.15) (width 1.524) (layer B.Cu) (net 23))
 (segment (start 168.91 53.34) (end 170.18 54.61) (width 1.524) (layer B.Cu) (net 23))
 (segment (start 164.465 53.34) (end 168.91 53.34) (width 1.524) (layer B.Cu) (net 23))
 (segment (start 162.56 51.435) (end 164.465 53.34) (width 1.524) (layer B.Cu) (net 23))
 (segment (start 162.56 48.895) (end 162.56 51.435) (width 1.524) (layer B.Cu) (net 23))
 (segment (start 157.48 43.815) (end 162.56 48.895) (width 1.524) (layer B.Cu) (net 23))
 (segment (start 111.125 43.815) (end 157.48 43.815) (width 1.524) (layer B.Cu) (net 23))
 (segment (start 109.22 45.72) (end 111.125 43.815) (width 1.524) (layer B.Cu) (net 23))
 (segment (start 109.22 62.865) (end 109.22 45.72) (width 1.524) (layer B.Cu) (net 23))
 (segment (start 111.76 65.405) (end 109.22 62.865) (width 1.524) (layer B.Cu) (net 23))
 (segment (start 163.195 60.325) (end 159.385 60.325) (width 1.524) (layer B.Cu) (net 23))
 (segment (start 156.21 63.5) (end 156.21 65.405) (width 1.524) (layer B.Cu) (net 23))
 (segment (start 159.385 60.325) (end 156.21 63.5) (width 1.524) (layer B.Cu) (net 23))
 (segment (start 133.35 65.405) (end 127.635 65.405) (width 1.524) (layer B.Cu) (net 16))
 (segment (start 122.555 70.485) (end 116.84 70.485) (width 1.524) (layer B.Cu) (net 16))
 (segment (start 127.635 65.405) (end 122.555 70.485) (width 1.524) (layer B.Cu) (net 16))
 (segment (start 116.84 74.295) (end 116.84 70.485) (width 1.524) (layer B.Cu) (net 16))
 (segment (start 167.64 50.8) (end 170.18 50.8) (width 1.524) (layer B.Cu) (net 22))
 (segment (start 172.085 52.705) (end 172.085 55.245) (width 1.524) (layer B.Cu) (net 22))
 (segment (start 170.18 50.8) (end 172.085 52.705) (width 1.524) (layer B.Cu) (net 22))
 (segment (start 172.085 58.42) (end 170.18 60.325) (width 1.524) (layer B.Cu) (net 22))
 (segment (start 172.085 55.245) (end 172.085 58.42) (width 1.524) (layer B.Cu) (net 22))
 (segment (start 167.64 62.865) (end 163.195 62.865) (width 1.524) (layer B.Cu) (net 22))
 (segment (start 170.18 60.325) (end 167.64 62.865) (width 1.524) (layer B.Cu) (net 22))
 (segment (start 113.03 47.625) (end 113.03 50.165) (width 0.3048) (layer B.Cu) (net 11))
 (segment (start 113.03 50.165) (end 113.03 52.705) (width 0.3048) (layer B.Cu) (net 11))
 (segment (start 113.03 52.705) (end 114.3 53.975) (width 0.3048) (layer B.Cu) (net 11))
 (segment (start 114.3 53.975) (end 114.3 59.055) (width 0.3048) (layer B.Cu) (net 11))
 (segment (start 114.3 59.055) (end 113.03 60.325) (width 0.3048) (layer B.Cu) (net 11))
 (segment (start 113.03 60.325) (end 120.015 60.325) (width 0.3048) (layer B.Cu) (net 11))
 (segment (start 127.635 97.79) (end 127.635 105.41) (width 0.3048) (layer B.Cu) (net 12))
 (segment (start 127.635 105.41) (end 143.51 121.285) (width 0.3048) (layer B.Cu) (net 12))
 (segment (start 127.635 90.17) (end 127.635 92.71) (width 0.3048) (layer B.Cu) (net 12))
 (segment (start 127.635 92.71) (end 125.73 94.615) (width 0.3048) (layer B.Cu) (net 12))
 (segment (start 125.73 94.615) (end 125.73 95.885) (width 0.3048) (layer B.Cu) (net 12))
 (segment (start 125.73 95.885) (end 127.635 97.79) (width 0.3048) (layer B.Cu) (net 12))
 (segment (start 143.51 70.485) (end 140.97 70.485) (width 0.3048) (layer B.Cu) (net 13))
 (segment (start 133.35 67.945) (end 129.54 67.945) (width 0.3048) (layer B.Cu) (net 14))
 (segment (start 133.35 62.865) (end 135.89 62.865) (width 1.524) (layer F.Cu) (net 17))
 (segment (start 138.43 65.405) (end 140.97 65.405) (width 1.524) (layer F.Cu) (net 17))
 (segment (start 135.89 62.865) (end 138.43 65.405) (width 1.524) (layer F.Cu) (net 17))
 (segment (start 121.92 84.455) (end 121.92 77.47) (width 1.524) (layer B.Cu) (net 17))
 (segment (start 138.43 121.285) (end 123.825 106.68) (width 1.524) (layer B.Cu) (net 17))
 (segment (start 121.92 104.775) (end 123.825 106.68) (width 1.524) (layer B.Cu) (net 17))
 (segment (start 121.92 84.455) (end 121.92 104.775) (width 1.524) (layer B.Cu) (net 17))
 (segment (start 127 62.865) (end 121.92 67.945) (width 1.524) (layer B.Cu) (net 17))
 (segment (start 128.27 62.865) (end 133.35 62.865) (width 1.524) (layer B.Cu) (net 17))
 (segment (start 128.27 62.865) (end 127 62.865) (width 1.524) (layer B.Cu) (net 17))
 (segment (start 140.97 65.405) (end 144.145 65.405) (width 1.524) (layer B.Cu) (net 17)))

